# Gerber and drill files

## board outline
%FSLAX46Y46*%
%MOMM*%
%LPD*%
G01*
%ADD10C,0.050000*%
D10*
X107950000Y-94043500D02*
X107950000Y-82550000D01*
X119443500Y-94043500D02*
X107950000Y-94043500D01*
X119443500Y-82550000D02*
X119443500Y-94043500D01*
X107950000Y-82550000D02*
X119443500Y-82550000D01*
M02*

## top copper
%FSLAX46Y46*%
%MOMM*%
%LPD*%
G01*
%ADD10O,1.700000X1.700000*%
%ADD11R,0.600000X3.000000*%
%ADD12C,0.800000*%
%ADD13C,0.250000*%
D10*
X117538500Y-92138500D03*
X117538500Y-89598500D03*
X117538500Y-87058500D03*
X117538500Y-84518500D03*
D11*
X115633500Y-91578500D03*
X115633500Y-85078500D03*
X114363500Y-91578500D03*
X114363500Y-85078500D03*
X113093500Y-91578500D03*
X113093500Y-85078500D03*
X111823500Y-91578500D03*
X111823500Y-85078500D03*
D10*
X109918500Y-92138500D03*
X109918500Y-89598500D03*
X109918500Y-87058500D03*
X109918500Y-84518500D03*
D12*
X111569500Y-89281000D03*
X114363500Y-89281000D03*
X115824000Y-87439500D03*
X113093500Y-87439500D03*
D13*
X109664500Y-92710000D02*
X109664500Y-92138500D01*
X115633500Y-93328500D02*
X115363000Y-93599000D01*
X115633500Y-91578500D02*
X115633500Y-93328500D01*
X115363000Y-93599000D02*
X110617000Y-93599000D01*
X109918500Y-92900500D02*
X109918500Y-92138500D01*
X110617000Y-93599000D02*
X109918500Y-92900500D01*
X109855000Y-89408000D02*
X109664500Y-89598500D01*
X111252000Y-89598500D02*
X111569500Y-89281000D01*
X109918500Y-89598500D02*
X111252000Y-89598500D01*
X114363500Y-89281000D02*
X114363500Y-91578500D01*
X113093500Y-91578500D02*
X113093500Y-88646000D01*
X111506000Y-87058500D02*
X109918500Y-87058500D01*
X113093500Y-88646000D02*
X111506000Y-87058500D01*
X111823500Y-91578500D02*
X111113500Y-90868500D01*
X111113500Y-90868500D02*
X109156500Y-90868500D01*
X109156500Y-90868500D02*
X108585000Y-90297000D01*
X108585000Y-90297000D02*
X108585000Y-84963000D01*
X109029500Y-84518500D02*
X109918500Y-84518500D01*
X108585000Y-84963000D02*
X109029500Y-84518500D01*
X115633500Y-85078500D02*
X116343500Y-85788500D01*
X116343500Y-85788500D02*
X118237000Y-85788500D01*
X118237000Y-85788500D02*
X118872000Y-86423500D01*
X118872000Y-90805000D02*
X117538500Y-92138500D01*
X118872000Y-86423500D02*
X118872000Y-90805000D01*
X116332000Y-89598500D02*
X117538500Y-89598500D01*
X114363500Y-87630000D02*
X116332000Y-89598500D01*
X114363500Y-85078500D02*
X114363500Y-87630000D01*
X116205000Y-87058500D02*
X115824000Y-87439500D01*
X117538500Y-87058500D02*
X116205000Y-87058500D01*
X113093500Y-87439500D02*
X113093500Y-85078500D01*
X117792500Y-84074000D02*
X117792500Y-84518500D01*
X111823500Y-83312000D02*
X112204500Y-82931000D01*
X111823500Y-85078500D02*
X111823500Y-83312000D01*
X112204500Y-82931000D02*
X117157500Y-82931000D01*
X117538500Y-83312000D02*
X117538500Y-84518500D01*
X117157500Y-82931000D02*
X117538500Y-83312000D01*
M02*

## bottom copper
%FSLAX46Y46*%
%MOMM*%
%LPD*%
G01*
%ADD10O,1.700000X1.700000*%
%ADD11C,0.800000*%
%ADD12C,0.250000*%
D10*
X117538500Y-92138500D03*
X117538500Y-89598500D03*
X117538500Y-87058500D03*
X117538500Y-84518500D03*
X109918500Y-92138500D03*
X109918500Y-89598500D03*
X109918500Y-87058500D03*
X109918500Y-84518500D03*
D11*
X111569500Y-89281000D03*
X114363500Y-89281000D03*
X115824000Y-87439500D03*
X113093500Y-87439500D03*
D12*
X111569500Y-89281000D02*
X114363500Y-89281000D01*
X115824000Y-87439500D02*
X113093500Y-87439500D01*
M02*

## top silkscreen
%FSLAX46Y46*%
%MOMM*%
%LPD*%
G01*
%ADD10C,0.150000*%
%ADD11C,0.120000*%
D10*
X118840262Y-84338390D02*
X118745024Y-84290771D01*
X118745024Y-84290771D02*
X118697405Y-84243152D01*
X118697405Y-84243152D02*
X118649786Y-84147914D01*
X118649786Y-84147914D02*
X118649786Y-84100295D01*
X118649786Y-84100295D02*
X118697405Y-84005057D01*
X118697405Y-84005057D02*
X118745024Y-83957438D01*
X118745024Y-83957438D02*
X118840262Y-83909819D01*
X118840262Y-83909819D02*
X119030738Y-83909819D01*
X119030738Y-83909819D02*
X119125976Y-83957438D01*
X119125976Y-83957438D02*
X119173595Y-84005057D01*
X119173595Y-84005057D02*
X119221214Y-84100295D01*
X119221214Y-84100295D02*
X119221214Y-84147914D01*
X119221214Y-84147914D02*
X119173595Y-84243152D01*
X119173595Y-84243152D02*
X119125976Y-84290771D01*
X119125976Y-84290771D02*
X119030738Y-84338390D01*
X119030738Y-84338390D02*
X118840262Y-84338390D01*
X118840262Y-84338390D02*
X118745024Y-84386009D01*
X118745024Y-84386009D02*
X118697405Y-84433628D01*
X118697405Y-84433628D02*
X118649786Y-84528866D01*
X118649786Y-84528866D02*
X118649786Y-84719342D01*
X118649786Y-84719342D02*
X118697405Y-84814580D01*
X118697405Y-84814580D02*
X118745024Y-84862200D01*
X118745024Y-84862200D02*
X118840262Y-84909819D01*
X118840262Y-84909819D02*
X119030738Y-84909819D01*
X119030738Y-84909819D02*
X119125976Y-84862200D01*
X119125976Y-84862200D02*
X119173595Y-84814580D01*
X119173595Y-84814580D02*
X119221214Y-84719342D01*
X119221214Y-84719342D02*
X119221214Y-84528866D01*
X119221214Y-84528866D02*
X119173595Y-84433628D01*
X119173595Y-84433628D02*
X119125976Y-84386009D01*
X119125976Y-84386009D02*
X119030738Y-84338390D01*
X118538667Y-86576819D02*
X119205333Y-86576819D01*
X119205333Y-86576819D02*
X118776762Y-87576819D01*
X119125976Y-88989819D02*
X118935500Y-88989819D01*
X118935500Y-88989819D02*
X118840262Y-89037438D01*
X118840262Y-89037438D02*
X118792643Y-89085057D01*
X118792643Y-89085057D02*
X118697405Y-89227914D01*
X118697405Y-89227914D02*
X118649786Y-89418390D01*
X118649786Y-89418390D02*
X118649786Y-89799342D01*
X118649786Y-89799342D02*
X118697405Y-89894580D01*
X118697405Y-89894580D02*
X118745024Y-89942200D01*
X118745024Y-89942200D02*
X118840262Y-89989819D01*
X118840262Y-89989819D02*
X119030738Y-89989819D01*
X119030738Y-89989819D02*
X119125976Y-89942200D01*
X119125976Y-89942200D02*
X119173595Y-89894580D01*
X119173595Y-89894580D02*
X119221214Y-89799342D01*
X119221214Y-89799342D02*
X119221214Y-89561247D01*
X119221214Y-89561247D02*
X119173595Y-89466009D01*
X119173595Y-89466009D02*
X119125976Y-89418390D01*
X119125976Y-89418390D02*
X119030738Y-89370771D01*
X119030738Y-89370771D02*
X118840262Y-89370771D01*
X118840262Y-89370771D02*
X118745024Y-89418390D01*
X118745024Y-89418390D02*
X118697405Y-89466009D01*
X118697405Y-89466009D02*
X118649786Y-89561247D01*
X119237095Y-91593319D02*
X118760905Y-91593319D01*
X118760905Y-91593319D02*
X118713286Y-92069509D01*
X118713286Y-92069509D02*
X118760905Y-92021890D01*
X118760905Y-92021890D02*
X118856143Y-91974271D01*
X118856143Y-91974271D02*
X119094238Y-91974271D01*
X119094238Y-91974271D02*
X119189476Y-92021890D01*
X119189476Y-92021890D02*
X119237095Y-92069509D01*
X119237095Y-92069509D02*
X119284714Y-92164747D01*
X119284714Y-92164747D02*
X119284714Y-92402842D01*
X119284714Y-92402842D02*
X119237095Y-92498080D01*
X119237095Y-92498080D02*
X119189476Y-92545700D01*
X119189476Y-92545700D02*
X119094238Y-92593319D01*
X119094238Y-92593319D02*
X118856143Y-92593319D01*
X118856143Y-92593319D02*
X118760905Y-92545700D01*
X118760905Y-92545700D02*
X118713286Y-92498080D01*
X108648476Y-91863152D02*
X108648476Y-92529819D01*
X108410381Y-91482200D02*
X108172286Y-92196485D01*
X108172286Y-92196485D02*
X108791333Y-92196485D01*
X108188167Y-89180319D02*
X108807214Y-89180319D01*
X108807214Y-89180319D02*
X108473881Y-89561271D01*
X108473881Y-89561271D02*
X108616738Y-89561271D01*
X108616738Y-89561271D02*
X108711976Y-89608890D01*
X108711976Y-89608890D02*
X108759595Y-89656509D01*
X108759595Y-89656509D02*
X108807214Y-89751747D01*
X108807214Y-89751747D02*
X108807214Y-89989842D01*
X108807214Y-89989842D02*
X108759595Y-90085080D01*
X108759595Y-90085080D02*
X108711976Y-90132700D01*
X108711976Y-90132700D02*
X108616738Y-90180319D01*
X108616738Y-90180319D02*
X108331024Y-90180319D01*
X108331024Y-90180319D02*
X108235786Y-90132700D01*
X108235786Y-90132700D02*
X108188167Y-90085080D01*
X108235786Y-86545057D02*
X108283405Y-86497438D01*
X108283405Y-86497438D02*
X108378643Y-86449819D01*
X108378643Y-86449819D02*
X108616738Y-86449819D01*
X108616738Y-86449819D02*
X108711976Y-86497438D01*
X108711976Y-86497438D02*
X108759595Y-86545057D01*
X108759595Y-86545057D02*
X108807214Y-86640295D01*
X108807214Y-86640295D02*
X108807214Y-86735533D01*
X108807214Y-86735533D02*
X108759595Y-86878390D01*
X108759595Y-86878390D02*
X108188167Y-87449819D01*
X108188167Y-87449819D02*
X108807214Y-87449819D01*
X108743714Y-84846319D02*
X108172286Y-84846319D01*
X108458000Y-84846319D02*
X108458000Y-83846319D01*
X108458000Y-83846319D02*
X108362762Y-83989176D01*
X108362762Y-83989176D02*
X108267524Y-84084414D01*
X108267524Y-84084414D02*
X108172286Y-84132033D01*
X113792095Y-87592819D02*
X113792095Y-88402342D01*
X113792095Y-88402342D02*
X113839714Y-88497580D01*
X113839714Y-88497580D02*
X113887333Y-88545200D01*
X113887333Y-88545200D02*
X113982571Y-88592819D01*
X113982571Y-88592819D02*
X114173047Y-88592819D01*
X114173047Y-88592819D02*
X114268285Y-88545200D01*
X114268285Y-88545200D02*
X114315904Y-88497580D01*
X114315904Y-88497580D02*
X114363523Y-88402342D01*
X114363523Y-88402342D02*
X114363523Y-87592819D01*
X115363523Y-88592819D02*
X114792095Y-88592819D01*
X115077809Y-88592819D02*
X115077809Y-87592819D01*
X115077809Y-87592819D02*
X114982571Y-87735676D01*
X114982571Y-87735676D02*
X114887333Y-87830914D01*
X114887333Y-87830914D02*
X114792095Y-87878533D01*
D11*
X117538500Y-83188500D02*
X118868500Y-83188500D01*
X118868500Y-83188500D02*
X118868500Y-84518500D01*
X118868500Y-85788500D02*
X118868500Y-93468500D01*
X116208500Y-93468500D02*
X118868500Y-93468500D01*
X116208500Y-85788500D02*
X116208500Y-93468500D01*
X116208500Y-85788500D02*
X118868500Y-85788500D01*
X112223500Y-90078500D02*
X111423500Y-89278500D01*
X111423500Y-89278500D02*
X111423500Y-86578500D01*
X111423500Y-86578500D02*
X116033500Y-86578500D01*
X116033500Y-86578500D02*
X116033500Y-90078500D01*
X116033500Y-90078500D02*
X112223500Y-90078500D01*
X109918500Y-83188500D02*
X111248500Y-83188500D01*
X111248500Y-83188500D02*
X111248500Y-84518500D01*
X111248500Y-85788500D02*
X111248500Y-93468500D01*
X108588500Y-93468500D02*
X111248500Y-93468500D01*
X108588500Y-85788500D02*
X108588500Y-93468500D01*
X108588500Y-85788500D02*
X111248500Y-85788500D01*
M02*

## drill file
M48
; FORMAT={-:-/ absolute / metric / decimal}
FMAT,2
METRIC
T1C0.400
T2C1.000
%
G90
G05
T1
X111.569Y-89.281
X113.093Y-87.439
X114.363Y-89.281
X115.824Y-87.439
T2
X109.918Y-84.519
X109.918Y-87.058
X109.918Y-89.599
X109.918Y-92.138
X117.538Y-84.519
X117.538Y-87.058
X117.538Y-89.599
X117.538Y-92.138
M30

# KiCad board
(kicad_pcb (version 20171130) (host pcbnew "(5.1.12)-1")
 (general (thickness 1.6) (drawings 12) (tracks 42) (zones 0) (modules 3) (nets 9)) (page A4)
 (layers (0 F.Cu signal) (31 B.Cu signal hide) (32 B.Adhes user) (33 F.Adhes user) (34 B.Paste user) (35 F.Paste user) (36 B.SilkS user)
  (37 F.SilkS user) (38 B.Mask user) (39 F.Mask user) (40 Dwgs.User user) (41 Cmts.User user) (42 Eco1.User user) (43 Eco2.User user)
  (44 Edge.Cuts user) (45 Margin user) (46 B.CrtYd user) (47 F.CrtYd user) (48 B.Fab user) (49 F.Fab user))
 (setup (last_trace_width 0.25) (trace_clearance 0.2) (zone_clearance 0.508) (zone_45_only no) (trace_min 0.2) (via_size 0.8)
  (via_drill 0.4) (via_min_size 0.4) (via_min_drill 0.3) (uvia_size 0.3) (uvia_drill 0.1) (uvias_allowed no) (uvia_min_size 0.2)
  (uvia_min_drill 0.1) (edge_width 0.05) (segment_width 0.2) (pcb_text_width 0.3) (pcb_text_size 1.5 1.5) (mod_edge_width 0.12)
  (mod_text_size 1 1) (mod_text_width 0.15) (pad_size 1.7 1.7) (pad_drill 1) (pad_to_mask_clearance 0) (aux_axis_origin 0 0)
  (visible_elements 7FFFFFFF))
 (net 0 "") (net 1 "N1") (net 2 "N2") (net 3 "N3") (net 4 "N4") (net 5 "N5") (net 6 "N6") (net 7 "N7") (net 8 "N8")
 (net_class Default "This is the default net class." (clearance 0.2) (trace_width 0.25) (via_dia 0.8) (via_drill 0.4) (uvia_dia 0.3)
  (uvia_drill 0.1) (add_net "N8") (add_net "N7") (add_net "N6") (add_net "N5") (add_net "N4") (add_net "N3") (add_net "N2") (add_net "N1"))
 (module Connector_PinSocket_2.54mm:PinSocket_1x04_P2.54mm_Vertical (layer F.Cu) (at 117.5385 84.5185)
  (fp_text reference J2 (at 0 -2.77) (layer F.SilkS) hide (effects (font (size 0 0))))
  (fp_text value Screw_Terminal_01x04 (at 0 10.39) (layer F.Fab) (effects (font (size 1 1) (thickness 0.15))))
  (fp_line (start 0 -1.33) (end 1.33 -1.33) (layer F.SilkS) (width 0.12))
  (fp_line (start 1.33 -1.33) (end 1.33 0) (layer F.SilkS) (width 0.12))
  (fp_line (start 1.33 1.27) (end 1.33 8.95) (layer F.SilkS) (width 0.12))
  (fp_line (start -1.33 8.95) (end 1.33 8.95) (layer F.SilkS) (width 0.12))
  (fp_line (start -1.33 1.27) (end -1.33 8.95) (layer F.SilkS) (width 0.12))
  (fp_line (start -1.33 1.27) (end 1.33 1.27) (layer F.SilkS) (width 0.12))
  (pad 4 thru_hole oval (at 0 7.62) (size 1.7 1.7) (drill 1) (layers *.Cu *.Mask) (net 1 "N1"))
  (pad 3 thru_hole oval (at 0 5.08) (size 1.7 1.7) (drill 1) (layers *.Cu *.Mask) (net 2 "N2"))
  (pad 2 thru_hole oval (at 0 2.54) (size 1.7 1.7) (drill 1) (layers *.Cu *.Mask) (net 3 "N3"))
  (pad 1 thru_hole oval (at 0 0) (size 1.7 1.7) (drill 1) (layers *.Cu *.Mask) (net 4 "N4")))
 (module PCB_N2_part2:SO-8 (layer F.Cu) (at 113.7285 88.3285)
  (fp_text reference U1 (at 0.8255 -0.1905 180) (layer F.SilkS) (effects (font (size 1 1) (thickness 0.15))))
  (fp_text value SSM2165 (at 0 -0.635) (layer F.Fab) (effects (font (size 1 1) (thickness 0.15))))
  (fp_line (start -1.505 1.75) (end -2.305 0.95) (layer F.SilkS) (width 0.12))
  (fp_line (start -2.305 0.95) (end -2.305 -1.75) (layer F.SilkS) (width 0.12))
  (fp_line (start -2.305 -1.75) (end 2.305 -1.75) (layer F.SilkS) (width 0.12))
  (fp_line (start 2.305 -1.75) (end 2.305 1.75) (layer F.SilkS) (width 0.12))
  (fp_line (start 2.305 1.75) (end -1.505 1.75) (layer F.SilkS) (width 0.12))
  (pad 4 smd rect (at 1.905 3.25) (size 0.6 3) (layers F.Cu F.Paste F.Mask) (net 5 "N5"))
  (pad 5 smd rect (at 1.905 -3.25) (size 0.6 3) (layers F.Cu F.Paste F.Mask) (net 1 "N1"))
  (pad 3 smd rect (at 0.635 3.25) (size 0.6 3) (layers F.Cu F.Paste F.Mask) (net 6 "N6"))
  (pad 6 smd rect (at 0.635 -3.25) (size 0.6 3) (layers F.Cu F.Paste F.Mask) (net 2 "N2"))
  (pad 2 smd rect (at -0.635 3.25) (size 0.6 3) (layers F.Cu F.Paste F.Mask) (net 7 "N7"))
  (pad 7 smd rect (at -0.635 -3.25) (size 0.6 3) (layers F.Cu F.Paste F.Mask) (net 3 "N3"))
  (pad 1 smd rect (at -1.905 3.25) (size 0.6 3) (layers F.Cu F.Paste F.Mask) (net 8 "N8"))
  (pad 8 smd rect (at -1.905 -3.25) (size 0.6 3) (layers F.Cu F.Paste F.Mask) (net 4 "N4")))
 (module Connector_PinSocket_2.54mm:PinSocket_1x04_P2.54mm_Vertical (layer F.Cu) (at 109.9185 84.5185)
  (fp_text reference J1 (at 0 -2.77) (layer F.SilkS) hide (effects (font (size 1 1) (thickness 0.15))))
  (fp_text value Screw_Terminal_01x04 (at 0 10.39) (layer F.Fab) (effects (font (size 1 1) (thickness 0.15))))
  (fp_line (start 0 -1.33) (end 1.33 -1.33) (layer F.SilkS) (width 0.12))
  (fp_line (start 1.33 -1.33) (end 1.33 0) (layer F.SilkS) (width 0.12))
  (fp_line (start 1.33 1.27) (end 1.33 8.95) (layer F.SilkS) (width 0.12))
  (fp_line (start -1.33 8.95) (end 1.33 8.95) (layer F.SilkS) (width 0.12))
  (fp_line (start -1.33 1.27) (end -1.33 8.95) (layer F.SilkS) (width 0.12))
  (fp_line (start -1.33 1.27) (end 1.33 1.27) (layer F.SilkS) (width 0.12))
  (pad 4 thru_hole oval (at 0 7.62) (size 1.7 1.7) (drill 1) (layers *.Cu *.Mask) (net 5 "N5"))
  (pad 3 thru_hole oval (at 0 5.08) (size 1.7 1.7) (drill 1) (layers *.Cu *.Mask) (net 6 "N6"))
  (pad 2 thru_hole oval (at 0 2.54) (size 1.7 1.7) (drill 1) (layers *.Cu *.Mask) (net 7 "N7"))
  (pad 1 thru_hole oval (at 0 0) (size 1.7 1.7) (drill 1) (layers *.Cu *.Mask) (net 8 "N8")))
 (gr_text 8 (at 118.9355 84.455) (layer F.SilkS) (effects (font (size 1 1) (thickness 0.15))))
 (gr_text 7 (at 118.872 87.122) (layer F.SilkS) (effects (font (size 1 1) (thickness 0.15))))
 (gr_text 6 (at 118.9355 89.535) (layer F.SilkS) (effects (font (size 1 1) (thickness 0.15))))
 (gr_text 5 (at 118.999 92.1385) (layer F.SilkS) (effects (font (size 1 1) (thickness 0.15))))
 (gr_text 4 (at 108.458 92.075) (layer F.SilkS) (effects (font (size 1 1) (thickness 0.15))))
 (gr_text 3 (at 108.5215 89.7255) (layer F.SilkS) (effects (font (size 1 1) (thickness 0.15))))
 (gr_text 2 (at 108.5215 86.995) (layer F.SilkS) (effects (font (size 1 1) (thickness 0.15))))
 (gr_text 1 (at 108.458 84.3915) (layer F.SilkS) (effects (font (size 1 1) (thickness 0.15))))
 (gr_line (start 107.95 94.0435) (end 107.95 82.55) (layer Edge.Cuts) (width 0.05))
 (gr_line (start 119.4435 94.0435) (end 107.95 94.0435) (layer Edge.Cuts) (width 0.05))
 (gr_line (start 119.4435 82.55) (end 119.4435 94.0435) (layer Edge.Cuts) (width 0.05))
 (gr_line (start 107.95 82.55) (end 119.4435 82.55) (layer Edge.Cuts) (width 0.05))
 (segment (start 109.6645 92.71) (end 109.6645 92.1385) (width 0.25) (layer F.Cu) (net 5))
 (segment (start 115.6335 93.3285) (end 115.363 93.599) (width 0.25) (layer F.Cu) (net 5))
 (segment (start 115.6335 91.5785) (end 115.6335 93.3285) (width 0.25) (layer F.Cu) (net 5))
 (segment (start 115.363 93.599) (end 110.617 93.599) (width 0.25) (layer F.Cu) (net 5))
 (segment (start 109.9185 92.9005) (end 109.9185 92.1385) (width 0.25) (layer F.Cu) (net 5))
 (segment (start 110.617 93.599) (end 109.9185 92.9005) (width 0.25) (layer F.Cu) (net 5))
 (segment (start 109.855 89.408) (end 109.6645 89.5985) (width 0.25) (layer F.Cu) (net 6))
 (via (at 111.5695 89.281) (size 0.8) (drill 0.4) (layers F.Cu B.Cu) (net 6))
 (segment (start 111.252 89.5985) (end 111.5695 89.281) (width 0.25) (layer F.Cu) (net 6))
 (segment (start 109.9185 89.5985) (end 111.252 89.5985) (width 0.25) (layer F.Cu) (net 6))
 (via (at 114.3635 89.281) (size 0.8) (drill 0.4) (layers F.Cu B.Cu) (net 6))
 (segment (start 111.5695 89.281) (end 114.3635 89.281) (width 0.25) (layer B.Cu) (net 6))
 (segment (start 114.3635 89.281) (end 114.3635 91.5785) (width 0.25) (layer F.Cu) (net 6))
 (segment (start 113.0935 91.5785) (end 113.0935 88.646) (width 0.25) (layer F.Cu) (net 7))
 (segment (start 111.506 87.0585) (end 109.9185 87.0585) (width 0.25) (layer F.Cu) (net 7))
 (segment (start 113.0935 88.646) (end 111.506 87.0585) (width 0.25) (layer F.Cu) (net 7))
 (segment (start 111.8235 91.5785) (end 111.1135 90.8685) (width 0.25) (layer F.Cu) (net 8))
 (segment (start 111.1135 90.8685) (end 109.1565 90.8685) (width 0.25) (layer F.Cu) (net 8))
 (segment (start 109.1565 90.8685) (end 108.585 90.297) (width 0.25) (layer F.Cu) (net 8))
 (segment (start 108.585 90.297) (end 108.585 84.963) (width 0.25) (layer F.Cu) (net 8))
 (segment (start 109.0295 84.5185) (end 109.9185 84.5185) (width 0.25) (layer F.Cu) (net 8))
 (segment (start 108.585 84.963) (end 109.0295 84.5185) (width 0.25) (layer F.Cu) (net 8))
 (segment (start 115.6335 85.0785) (end 116.3435 85.7885) (width 0.25) (layer F.Cu) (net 1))
 (segment (start 116.3435 85.7885) (end 118.237 85.7885) (width 0.25) (layer F.Cu) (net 1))
 (segment (start 118.237 85.7885) (end 118.872 86.4235) (width 0.25) (layer F.Cu) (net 1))
 (segment (start 118.872 90.805) (end 117.5385 92.1385) (width 0.25) (layer F.Cu) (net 1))
 (segment (start 118.872 86.4235) (end 118.872 90.805) (width 0.25) (layer F.Cu) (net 1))
 (segment (start 116.332 89.5985) (end 117.5385 89.5985) (width 0.25) (layer F.Cu) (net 2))
 (segment (start 114.3635 87.63) (end 116.332 89.5985) (width 0.25) (layer F.Cu) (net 2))
 (segment (start 114.3635 85.0785) (end 114.3635 87.63) (width 0.25) (layer F.Cu) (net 2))
 (via (at 115.824 87.4395) (size 0.8) (drill 0.4) (layers F.Cu B.Cu) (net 3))
 (segment (start 116.205 87.0585) (end 115.824 87.4395) (width 0.25) (layer F.Cu) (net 3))
 (segment (start 117.5385 87.0585) (end 116.205 87.0585) (width 0.25) (layer F.Cu) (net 3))
 (via (at 113.0935 87.4395) (size 0.8) (drill 0.4) (layers F.Cu B.Cu) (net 3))
 (segment (start 115.824 87.4395) (end 113.0935 87.4395) (width 0.25) (layer B.Cu) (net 3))
 (segment (start 113.0935 87.4395) (end 113.0935 85.0785) (width 0.25) (layer F.Cu) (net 3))
 (segment (start 117.7925 84.074) (end 117.7925 84.5185) (width 0.25) (layer F.Cu) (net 4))
 (segment (start 111.8235 83.312) (end 112.2045 82.931) (width 0.25) (layer F.Cu) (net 4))
 (segment (start 111.8235 85.0785) (end 111.8235 83.312) (width 0.25) (layer F.Cu) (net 4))
 (segment (start 112.2045 82.931) (end 117.1575 82.931) (width 0.25) (layer F.Cu) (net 4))
 (segment (start 117.5385 83.312) (end 117.5385 84.5185) (width 0.25) (layer F.Cu) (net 4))
 (segment (start 117.1575 82.931) (end 117.5385 83.312) (width 0.25) (layer F.Cu) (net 4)))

